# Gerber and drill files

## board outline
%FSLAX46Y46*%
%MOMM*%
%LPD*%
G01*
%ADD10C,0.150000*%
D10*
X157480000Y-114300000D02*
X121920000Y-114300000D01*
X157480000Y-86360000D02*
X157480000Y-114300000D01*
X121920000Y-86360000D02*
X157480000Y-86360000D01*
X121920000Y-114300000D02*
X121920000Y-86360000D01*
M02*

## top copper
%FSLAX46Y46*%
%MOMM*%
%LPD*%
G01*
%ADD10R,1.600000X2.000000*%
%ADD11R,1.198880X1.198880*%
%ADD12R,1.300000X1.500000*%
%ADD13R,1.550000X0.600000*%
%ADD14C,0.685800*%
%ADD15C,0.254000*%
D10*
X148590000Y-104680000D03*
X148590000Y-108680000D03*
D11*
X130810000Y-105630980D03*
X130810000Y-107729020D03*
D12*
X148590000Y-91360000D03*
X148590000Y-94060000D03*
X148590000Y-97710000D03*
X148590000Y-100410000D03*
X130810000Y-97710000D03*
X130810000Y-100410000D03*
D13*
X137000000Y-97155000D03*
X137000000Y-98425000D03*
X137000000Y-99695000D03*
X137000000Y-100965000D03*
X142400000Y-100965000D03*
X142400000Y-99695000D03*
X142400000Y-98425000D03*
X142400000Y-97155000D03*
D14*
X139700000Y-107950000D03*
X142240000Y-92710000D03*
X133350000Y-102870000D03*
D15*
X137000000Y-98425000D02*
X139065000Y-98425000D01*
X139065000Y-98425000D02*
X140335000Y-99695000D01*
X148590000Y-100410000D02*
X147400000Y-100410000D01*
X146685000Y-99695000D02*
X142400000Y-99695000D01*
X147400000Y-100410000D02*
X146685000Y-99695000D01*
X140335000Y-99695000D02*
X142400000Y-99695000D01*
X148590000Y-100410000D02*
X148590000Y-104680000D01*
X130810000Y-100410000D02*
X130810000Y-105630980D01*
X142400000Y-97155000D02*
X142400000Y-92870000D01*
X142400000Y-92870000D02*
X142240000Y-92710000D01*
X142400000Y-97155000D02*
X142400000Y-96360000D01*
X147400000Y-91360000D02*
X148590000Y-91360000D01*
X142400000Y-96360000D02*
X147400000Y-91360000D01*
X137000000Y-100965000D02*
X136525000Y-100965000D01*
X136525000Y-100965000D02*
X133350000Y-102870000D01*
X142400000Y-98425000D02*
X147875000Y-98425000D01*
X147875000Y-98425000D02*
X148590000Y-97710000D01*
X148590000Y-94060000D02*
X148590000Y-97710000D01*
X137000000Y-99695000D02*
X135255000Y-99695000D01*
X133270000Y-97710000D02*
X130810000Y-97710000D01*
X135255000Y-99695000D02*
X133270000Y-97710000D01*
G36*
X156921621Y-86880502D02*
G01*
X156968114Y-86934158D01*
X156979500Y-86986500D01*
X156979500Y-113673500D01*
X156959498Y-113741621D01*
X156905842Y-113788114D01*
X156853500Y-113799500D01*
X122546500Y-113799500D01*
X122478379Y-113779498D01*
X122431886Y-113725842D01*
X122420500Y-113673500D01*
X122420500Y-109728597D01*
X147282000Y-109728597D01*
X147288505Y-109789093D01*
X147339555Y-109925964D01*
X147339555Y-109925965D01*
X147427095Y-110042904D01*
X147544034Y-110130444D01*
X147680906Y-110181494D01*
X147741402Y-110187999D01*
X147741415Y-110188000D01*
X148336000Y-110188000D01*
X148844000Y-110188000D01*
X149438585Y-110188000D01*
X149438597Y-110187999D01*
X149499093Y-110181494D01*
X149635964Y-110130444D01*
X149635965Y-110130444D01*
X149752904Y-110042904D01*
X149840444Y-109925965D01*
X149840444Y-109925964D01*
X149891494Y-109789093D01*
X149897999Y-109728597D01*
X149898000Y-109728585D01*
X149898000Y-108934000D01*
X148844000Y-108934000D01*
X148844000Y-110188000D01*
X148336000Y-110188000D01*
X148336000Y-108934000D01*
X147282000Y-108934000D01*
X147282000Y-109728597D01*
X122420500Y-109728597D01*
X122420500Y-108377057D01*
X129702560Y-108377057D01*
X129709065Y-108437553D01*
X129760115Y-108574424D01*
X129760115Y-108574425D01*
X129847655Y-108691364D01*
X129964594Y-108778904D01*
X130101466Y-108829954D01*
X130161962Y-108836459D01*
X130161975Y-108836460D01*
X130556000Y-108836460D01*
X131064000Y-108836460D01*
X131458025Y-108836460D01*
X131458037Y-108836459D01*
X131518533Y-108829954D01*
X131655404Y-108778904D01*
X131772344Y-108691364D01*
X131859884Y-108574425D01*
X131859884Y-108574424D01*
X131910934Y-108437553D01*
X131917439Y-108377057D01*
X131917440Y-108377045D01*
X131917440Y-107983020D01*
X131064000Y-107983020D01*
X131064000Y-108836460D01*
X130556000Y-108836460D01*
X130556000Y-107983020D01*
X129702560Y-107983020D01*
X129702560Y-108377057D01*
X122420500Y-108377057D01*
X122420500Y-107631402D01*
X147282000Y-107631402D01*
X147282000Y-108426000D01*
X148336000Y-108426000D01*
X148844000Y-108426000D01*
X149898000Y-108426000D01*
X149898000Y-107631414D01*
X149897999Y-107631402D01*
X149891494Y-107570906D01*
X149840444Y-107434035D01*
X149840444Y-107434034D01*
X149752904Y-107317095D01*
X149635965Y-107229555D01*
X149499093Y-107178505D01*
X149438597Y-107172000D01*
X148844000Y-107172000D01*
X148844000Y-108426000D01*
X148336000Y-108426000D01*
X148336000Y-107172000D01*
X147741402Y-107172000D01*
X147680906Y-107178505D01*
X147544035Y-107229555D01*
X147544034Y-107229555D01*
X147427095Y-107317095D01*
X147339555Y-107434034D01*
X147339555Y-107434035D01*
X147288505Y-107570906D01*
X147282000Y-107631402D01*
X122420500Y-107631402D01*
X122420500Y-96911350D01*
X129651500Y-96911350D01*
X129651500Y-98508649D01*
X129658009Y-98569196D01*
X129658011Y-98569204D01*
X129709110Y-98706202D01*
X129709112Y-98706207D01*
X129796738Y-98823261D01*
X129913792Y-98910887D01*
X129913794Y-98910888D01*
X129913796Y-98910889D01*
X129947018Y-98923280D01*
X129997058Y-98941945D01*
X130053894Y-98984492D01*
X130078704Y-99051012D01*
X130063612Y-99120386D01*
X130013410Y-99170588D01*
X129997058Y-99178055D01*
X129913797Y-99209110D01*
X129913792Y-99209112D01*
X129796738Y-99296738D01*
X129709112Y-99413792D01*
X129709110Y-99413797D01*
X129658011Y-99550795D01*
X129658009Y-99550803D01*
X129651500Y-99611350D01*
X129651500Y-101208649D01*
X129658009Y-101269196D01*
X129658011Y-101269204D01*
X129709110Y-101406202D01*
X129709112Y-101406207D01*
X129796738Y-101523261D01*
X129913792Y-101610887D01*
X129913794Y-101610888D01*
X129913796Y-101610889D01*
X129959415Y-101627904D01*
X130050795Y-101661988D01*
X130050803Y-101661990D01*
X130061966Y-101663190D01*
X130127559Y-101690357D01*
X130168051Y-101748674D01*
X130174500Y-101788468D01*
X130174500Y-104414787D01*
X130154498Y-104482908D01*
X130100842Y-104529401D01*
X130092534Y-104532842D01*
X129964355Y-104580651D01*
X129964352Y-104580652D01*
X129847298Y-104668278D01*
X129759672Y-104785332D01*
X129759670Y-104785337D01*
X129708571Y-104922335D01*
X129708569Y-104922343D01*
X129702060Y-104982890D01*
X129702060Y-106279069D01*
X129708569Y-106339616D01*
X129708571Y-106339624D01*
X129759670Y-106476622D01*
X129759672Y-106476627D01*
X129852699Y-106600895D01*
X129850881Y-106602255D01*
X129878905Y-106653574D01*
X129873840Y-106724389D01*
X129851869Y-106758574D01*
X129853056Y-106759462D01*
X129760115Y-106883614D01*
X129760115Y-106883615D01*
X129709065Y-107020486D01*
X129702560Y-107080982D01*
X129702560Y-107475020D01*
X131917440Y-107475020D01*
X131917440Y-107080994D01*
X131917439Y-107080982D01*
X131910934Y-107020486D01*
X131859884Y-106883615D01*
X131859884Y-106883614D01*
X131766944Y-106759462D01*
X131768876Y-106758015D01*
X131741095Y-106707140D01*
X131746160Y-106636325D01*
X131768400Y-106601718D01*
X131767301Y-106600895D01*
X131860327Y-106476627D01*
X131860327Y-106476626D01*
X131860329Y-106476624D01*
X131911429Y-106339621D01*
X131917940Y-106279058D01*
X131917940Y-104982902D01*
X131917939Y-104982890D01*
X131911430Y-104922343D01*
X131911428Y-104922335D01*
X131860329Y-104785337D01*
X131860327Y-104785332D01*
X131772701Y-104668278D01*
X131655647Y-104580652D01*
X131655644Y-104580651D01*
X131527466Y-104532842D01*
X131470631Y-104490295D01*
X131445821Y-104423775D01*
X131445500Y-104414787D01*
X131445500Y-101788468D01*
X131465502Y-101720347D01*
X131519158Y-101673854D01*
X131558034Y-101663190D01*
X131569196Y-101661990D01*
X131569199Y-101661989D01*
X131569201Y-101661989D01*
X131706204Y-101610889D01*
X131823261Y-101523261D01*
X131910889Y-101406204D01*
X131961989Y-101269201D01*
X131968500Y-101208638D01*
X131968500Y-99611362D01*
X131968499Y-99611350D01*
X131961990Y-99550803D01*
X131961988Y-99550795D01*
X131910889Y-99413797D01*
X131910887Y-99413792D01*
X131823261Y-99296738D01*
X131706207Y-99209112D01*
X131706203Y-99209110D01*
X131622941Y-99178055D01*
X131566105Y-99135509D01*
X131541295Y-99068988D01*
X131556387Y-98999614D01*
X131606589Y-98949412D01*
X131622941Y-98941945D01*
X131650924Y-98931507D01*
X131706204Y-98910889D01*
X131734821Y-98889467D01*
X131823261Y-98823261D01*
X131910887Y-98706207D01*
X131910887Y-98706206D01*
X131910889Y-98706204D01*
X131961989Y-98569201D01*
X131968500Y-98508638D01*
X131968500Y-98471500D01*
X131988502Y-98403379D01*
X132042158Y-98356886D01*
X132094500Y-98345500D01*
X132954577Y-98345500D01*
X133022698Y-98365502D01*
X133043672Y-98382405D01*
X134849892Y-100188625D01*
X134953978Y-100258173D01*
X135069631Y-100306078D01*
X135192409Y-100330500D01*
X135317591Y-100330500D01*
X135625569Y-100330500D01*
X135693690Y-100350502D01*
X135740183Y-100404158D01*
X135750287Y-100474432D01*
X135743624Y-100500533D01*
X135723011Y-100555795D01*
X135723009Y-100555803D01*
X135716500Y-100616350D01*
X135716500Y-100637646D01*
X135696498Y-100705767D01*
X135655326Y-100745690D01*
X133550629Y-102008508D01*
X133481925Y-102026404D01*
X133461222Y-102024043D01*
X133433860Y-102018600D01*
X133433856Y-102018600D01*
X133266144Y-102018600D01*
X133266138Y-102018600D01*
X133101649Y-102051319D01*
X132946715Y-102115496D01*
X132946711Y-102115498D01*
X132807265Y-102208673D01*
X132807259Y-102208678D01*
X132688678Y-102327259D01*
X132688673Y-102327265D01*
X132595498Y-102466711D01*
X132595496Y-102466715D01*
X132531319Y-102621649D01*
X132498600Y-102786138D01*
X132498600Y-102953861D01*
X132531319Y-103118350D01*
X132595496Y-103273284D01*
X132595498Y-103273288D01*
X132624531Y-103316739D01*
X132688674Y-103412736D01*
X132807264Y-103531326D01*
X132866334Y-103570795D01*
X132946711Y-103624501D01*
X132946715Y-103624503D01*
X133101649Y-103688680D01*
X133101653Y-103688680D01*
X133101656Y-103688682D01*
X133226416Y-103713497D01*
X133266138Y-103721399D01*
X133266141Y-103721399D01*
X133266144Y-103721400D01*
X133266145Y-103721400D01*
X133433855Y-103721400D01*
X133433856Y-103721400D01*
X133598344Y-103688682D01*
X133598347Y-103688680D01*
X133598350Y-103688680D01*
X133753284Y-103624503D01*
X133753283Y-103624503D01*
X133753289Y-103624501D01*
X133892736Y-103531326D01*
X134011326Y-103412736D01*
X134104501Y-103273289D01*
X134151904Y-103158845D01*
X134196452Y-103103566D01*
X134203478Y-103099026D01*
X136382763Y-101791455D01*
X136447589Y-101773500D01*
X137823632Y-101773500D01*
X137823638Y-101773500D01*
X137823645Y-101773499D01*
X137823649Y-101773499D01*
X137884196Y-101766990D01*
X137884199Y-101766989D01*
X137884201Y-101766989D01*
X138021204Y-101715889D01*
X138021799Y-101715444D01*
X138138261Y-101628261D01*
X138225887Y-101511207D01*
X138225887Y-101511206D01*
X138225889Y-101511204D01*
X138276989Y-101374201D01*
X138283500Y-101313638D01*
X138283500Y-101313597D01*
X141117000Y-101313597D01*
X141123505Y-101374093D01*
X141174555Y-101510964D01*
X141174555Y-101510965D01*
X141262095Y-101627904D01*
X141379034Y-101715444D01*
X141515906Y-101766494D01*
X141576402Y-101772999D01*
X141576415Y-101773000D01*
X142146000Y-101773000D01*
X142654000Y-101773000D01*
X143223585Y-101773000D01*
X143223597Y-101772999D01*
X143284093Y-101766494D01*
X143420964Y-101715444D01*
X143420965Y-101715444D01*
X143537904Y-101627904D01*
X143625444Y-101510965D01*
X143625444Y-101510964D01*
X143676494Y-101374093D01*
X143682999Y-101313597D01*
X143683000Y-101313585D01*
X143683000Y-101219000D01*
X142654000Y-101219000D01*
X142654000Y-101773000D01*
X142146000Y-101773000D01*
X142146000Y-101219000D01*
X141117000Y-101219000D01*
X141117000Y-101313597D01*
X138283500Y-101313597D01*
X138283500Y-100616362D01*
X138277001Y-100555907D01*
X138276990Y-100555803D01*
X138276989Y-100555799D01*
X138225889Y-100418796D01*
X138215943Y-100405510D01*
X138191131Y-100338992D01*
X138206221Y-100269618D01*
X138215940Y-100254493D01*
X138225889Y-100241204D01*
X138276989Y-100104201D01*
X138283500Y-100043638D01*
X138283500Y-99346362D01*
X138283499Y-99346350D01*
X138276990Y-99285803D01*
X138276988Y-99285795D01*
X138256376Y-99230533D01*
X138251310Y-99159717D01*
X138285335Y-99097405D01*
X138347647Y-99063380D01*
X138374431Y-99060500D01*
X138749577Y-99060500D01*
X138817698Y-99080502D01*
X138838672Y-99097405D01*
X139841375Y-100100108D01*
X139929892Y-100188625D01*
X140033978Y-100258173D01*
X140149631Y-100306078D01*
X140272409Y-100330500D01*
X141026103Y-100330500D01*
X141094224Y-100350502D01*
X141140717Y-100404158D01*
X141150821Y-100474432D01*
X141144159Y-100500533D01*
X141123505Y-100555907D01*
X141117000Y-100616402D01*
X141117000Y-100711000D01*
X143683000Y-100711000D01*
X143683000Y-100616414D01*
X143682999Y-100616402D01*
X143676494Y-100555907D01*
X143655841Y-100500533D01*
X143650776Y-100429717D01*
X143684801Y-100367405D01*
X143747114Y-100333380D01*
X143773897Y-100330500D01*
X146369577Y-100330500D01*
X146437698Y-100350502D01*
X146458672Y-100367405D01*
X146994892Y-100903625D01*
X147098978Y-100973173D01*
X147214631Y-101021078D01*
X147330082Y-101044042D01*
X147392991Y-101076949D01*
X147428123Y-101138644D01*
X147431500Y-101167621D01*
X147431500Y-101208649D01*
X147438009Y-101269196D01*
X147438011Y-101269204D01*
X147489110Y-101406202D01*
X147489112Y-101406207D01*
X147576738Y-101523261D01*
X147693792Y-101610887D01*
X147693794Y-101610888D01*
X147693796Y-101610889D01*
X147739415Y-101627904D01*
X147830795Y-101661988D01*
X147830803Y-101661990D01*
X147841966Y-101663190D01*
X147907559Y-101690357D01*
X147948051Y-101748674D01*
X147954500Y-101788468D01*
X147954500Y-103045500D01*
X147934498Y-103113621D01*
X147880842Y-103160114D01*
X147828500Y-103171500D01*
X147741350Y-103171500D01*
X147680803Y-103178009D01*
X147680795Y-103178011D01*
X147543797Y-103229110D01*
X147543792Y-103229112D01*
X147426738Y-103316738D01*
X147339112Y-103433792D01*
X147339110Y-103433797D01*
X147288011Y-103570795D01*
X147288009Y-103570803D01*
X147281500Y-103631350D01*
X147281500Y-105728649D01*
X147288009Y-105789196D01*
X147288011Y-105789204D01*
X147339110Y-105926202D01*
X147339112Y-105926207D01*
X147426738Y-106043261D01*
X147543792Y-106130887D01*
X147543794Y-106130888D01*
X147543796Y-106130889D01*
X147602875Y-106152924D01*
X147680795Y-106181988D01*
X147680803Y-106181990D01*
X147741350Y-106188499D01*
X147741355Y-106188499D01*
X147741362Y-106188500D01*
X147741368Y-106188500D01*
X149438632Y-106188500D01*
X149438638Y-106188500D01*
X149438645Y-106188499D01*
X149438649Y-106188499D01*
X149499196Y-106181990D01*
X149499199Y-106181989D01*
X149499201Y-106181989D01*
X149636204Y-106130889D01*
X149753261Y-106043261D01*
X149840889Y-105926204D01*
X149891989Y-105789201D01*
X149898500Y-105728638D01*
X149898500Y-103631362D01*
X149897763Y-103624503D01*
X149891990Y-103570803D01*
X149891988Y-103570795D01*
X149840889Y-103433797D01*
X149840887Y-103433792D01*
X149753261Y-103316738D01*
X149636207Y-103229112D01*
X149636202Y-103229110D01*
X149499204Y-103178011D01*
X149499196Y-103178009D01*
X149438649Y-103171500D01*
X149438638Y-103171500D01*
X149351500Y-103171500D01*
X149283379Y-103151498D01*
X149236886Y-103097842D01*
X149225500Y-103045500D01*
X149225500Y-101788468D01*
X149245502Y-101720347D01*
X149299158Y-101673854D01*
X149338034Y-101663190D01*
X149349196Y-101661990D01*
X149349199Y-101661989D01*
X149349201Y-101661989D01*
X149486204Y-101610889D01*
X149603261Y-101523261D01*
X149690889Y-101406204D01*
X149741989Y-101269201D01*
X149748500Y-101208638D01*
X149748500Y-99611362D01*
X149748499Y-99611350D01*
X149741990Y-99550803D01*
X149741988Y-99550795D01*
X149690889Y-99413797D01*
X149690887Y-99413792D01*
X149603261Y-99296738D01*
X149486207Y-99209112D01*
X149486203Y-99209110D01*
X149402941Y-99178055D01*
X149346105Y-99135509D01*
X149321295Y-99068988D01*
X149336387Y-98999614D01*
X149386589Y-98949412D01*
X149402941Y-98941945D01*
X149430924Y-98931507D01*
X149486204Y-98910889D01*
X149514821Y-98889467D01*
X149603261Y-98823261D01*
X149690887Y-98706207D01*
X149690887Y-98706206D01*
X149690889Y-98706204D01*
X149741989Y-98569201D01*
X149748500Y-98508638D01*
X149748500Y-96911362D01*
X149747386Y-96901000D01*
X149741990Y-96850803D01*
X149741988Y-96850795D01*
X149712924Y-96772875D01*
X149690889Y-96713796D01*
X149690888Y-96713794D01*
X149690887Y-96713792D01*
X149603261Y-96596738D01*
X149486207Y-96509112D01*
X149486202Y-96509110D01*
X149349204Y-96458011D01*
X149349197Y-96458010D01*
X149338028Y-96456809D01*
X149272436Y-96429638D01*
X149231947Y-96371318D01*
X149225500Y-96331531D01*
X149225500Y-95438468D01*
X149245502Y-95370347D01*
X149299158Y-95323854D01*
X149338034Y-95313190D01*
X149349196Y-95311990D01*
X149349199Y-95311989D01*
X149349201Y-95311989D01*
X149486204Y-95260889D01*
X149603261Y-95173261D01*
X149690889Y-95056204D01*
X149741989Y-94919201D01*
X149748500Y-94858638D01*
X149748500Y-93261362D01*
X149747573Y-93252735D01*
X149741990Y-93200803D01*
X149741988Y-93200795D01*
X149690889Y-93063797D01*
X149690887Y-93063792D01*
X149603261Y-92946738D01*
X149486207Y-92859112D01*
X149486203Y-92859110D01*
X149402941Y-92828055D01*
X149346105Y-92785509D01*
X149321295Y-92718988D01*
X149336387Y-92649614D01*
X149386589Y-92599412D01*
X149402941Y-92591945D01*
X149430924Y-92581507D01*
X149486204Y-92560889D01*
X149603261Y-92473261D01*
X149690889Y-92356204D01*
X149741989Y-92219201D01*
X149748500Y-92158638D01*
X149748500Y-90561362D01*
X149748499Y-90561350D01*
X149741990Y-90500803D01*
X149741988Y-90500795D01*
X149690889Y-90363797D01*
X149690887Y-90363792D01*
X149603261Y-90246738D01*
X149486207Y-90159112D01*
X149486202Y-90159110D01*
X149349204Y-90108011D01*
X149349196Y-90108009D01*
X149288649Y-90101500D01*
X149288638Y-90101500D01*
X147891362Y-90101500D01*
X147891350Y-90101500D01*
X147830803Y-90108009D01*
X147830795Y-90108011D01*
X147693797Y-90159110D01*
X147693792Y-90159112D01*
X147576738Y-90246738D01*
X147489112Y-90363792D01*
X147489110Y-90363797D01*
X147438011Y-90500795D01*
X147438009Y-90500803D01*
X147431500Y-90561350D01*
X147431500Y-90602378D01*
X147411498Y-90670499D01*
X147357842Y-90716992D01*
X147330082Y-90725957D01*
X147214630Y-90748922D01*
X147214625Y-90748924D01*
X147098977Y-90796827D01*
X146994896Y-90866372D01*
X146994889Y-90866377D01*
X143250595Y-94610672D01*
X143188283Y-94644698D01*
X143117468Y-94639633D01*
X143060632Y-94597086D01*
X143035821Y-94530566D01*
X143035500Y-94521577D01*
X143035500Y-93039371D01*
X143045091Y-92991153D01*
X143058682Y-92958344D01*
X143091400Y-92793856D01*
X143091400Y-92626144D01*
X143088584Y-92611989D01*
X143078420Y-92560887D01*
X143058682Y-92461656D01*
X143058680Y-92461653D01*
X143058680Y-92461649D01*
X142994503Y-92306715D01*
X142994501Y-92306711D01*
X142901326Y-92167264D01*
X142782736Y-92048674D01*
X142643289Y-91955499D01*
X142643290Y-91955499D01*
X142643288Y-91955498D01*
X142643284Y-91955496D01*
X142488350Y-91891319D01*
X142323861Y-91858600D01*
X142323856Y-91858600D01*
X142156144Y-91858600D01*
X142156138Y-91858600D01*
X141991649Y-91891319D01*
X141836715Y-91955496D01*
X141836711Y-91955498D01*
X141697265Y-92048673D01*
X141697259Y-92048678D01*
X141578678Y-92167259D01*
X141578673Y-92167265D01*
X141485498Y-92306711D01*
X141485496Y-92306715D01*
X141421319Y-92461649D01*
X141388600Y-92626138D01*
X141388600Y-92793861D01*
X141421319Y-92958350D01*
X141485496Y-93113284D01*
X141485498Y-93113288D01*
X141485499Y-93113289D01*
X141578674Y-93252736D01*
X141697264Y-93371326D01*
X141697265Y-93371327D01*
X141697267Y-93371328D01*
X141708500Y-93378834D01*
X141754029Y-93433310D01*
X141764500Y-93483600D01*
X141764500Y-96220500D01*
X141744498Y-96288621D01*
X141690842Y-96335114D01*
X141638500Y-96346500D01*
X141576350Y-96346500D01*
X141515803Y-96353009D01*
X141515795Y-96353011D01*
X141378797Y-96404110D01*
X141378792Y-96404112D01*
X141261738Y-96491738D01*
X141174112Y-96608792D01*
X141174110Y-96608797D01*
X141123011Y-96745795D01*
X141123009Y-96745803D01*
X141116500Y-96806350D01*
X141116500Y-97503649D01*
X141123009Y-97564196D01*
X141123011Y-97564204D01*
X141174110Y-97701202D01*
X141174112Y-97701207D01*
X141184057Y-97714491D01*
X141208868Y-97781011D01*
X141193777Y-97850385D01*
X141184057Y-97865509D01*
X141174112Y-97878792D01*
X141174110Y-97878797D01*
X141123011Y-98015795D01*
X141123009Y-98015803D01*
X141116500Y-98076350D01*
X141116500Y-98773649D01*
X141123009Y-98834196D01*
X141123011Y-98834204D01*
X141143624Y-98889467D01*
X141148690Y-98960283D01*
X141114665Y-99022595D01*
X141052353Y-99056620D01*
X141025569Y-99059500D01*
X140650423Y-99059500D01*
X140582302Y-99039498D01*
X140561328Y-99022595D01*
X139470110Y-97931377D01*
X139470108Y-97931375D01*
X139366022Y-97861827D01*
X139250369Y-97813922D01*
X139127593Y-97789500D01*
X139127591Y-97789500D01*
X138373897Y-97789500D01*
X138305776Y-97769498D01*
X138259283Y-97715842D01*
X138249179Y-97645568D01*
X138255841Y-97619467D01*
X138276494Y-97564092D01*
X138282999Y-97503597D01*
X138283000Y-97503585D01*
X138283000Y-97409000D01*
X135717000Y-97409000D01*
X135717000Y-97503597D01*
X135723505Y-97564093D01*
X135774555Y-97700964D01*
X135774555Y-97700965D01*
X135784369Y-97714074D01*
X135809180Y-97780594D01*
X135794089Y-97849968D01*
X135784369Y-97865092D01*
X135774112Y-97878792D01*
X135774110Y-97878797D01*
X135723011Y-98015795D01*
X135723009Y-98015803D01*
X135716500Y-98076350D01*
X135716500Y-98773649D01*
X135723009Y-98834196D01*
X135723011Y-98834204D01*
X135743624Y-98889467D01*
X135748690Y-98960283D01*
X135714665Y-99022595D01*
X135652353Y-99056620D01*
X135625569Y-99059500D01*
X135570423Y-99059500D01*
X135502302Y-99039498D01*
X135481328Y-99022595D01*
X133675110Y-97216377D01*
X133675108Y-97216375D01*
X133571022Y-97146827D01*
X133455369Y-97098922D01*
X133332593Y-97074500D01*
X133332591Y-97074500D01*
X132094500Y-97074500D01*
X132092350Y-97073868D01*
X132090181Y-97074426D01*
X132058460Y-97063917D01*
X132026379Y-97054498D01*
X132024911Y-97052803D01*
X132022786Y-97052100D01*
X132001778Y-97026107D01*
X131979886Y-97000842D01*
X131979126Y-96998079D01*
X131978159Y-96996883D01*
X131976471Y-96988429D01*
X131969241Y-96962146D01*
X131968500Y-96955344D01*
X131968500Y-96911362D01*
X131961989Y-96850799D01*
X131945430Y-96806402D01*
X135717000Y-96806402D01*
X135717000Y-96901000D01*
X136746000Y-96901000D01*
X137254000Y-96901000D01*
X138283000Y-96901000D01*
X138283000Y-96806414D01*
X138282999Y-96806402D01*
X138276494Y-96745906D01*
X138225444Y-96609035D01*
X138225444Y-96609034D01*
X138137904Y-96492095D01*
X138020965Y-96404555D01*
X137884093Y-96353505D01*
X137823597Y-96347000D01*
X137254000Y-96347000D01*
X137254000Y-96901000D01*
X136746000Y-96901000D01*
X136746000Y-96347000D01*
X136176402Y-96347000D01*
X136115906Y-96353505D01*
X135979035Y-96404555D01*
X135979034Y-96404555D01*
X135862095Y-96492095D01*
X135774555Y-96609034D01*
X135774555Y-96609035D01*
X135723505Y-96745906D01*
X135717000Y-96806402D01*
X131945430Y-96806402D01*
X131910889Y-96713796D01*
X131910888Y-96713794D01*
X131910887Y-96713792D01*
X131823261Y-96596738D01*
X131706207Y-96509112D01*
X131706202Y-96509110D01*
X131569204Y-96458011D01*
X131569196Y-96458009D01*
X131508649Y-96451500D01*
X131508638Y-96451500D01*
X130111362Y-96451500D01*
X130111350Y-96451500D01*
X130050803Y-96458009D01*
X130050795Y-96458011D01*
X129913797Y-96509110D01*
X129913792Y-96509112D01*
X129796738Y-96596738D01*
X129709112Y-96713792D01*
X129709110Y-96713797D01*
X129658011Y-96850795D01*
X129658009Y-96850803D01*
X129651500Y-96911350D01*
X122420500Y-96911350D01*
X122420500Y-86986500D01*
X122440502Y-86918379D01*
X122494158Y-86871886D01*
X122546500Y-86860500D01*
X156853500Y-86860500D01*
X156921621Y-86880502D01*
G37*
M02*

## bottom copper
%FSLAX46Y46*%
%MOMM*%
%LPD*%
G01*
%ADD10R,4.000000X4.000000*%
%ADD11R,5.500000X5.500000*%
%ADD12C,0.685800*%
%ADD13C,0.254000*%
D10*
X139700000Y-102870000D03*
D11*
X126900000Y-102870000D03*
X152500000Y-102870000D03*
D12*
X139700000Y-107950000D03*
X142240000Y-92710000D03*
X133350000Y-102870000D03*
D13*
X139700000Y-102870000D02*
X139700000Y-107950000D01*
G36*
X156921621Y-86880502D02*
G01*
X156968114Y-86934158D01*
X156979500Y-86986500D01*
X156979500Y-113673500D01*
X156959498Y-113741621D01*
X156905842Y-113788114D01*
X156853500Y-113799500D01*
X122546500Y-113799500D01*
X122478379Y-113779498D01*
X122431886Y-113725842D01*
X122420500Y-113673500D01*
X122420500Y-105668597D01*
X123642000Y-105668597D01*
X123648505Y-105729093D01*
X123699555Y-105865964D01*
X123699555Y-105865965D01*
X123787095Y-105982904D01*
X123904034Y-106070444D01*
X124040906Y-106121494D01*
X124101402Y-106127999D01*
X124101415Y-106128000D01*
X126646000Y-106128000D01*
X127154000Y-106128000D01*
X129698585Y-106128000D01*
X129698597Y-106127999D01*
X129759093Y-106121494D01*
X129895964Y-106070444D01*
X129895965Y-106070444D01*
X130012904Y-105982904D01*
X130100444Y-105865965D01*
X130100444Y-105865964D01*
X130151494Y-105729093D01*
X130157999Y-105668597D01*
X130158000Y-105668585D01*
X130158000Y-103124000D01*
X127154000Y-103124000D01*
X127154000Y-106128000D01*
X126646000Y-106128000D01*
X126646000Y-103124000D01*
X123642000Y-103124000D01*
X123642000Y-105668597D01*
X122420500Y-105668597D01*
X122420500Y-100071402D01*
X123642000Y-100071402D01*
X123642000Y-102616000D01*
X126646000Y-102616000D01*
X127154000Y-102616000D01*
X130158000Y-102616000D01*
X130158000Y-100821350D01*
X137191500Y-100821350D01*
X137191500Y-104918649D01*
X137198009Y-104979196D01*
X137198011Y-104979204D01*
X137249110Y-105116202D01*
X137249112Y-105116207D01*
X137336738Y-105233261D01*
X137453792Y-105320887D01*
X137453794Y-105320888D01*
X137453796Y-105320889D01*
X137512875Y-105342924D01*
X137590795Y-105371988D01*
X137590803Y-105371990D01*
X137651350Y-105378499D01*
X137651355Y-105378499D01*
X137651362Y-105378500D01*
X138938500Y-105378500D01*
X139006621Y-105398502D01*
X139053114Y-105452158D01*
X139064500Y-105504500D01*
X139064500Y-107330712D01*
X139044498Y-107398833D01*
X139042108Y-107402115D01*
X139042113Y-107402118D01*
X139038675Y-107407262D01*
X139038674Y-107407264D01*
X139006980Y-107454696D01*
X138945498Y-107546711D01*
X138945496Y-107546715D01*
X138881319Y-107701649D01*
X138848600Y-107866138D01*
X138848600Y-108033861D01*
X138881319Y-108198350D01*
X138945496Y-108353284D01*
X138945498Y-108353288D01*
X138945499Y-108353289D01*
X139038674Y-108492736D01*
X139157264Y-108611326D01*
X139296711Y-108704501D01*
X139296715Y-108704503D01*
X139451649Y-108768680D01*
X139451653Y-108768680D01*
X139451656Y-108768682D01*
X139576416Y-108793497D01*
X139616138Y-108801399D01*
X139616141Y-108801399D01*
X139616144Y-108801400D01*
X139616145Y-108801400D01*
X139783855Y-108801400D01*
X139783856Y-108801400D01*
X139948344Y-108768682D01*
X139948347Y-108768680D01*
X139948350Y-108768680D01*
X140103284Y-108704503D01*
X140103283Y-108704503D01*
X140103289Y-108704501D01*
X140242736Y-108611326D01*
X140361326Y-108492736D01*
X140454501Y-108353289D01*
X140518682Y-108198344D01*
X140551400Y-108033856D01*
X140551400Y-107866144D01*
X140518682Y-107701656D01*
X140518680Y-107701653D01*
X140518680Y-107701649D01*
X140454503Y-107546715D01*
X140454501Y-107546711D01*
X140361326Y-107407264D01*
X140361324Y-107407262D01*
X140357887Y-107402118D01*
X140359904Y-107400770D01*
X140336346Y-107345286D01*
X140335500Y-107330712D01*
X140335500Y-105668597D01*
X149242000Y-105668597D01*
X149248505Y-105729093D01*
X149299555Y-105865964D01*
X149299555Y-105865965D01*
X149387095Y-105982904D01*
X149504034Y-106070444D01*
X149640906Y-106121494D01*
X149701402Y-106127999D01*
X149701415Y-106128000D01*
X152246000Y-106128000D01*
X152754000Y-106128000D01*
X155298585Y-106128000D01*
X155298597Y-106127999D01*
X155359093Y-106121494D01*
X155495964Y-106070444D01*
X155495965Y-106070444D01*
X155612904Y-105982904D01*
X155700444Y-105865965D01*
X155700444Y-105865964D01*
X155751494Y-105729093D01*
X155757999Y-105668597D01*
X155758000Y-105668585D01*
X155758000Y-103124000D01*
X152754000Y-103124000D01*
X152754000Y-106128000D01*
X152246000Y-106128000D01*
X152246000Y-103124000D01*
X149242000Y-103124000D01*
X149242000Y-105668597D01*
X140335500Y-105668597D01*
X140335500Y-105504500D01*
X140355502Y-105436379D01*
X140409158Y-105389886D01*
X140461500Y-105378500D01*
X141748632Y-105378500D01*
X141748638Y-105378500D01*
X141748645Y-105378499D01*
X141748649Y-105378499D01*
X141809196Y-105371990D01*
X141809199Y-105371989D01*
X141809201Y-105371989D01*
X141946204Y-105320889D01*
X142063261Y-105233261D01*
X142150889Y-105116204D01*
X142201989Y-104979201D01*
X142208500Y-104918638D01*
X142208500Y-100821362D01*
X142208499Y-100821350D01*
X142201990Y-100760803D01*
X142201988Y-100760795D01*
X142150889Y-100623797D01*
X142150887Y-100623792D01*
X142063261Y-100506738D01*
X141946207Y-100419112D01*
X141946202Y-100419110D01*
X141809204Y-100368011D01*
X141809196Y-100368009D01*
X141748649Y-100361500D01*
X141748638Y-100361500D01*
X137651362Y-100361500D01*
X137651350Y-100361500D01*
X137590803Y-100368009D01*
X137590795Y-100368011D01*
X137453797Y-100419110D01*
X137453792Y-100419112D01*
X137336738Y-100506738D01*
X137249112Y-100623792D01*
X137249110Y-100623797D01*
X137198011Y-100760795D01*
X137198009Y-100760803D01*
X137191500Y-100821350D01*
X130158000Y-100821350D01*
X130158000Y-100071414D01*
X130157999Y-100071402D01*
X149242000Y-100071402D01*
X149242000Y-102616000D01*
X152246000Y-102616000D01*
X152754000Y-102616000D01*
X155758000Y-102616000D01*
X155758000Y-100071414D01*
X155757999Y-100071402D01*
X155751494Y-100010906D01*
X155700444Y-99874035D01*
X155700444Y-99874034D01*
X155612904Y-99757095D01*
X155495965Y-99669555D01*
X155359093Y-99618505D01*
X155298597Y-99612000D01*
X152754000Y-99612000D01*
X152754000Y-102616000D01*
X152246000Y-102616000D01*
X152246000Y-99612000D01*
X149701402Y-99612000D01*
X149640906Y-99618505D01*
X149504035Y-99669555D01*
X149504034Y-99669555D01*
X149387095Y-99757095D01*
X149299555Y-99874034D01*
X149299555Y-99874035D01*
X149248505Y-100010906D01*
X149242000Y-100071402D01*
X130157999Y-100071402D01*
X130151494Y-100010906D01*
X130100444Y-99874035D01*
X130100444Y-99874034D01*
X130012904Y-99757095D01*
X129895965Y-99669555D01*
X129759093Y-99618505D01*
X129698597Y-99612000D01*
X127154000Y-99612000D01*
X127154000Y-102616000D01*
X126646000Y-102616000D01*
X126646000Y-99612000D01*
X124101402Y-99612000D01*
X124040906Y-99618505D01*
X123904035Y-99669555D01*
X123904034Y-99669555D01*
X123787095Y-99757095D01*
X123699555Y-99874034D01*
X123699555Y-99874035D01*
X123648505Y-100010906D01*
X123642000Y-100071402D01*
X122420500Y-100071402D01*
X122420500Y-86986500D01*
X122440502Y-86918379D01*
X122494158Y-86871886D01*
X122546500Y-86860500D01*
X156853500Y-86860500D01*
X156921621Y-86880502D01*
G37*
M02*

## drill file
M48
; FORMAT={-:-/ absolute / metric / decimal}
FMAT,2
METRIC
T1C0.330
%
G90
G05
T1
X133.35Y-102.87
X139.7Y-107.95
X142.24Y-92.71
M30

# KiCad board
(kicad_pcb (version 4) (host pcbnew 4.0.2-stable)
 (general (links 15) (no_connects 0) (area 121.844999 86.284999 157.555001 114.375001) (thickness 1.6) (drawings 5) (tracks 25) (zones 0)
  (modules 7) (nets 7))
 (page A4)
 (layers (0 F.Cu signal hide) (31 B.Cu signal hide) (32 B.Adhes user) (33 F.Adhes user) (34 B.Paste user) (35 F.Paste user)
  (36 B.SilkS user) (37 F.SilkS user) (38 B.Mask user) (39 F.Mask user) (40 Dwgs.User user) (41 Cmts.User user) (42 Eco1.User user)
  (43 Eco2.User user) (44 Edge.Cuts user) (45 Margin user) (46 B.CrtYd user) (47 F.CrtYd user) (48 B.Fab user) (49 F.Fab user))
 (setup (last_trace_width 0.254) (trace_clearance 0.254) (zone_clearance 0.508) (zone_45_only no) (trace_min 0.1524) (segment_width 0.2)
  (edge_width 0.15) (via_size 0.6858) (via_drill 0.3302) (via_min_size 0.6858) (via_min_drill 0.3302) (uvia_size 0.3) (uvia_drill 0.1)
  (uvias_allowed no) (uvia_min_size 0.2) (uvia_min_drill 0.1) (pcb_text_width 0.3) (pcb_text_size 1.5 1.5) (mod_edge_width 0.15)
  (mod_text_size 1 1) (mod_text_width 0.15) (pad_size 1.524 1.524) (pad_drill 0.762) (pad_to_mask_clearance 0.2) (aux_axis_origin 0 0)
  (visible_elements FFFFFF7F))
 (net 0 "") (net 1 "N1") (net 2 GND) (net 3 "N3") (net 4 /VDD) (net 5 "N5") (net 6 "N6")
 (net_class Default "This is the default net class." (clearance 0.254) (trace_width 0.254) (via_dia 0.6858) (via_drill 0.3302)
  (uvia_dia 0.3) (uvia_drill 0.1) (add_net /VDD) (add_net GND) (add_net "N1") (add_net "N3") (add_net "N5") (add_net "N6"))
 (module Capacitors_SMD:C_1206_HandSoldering (layer F.Cu) (at 148.59 106.68 270)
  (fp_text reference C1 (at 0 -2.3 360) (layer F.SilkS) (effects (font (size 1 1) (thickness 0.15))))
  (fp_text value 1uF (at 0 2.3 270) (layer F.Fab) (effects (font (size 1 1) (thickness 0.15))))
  (pad 1 smd rect (at -2 0 270) (size 2 1.6) (layers F.Cu F.Paste F.Mask) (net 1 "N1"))
  (pad 2 smd rect (at 2 0 270) (size 2 1.6) (layers F.Cu F.Paste F.Mask) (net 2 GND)))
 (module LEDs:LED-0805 (layer F.Cu) (at 130.81 106.68 90)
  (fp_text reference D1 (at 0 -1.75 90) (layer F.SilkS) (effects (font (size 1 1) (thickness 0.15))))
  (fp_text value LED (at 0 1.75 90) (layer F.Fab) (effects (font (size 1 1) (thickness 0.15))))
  (pad 2 smd rect (at 1.04902 0 270) (size 1.19888 1.19888) (layers F.Cu F.Paste F.Mask) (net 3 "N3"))
  (pad 1 smd rect (at -1.04902 0 270) (size 1.19888 1.19888) (layers F.Cu F.Paste F.Mask) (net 2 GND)))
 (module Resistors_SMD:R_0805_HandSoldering (layer F.Cu) (at 148.59 92.71 270)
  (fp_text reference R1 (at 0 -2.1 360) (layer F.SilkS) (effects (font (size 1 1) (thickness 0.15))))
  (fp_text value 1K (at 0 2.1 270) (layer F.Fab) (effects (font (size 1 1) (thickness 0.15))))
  (pad 1 smd rect (at -1.35 0 270) (size 1.5 1.3) (layers F.Cu F.Paste F.Mask) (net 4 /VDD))
  (pad 2 smd rect (at 1.35 0 270) (size 1.5 1.3) (layers F.Cu F.Paste F.Mask) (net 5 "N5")))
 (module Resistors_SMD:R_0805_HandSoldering (layer F.Cu) (at 148.59 99.06 270)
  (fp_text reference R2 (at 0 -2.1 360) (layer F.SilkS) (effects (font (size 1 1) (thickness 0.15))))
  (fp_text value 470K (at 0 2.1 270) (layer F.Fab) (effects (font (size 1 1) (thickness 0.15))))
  (pad 1 smd rect (at -1.35 0 270) (size 1.5 1.3) (layers F.Cu F.Paste F.Mask) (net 5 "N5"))
  (pad 2 smd rect (at 1.35 0 270) (size 1.5 1.3) (layers F.Cu F.Paste F.Mask) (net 1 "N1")))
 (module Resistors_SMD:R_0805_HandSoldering (layer F.Cu) (at 130.81 99.06 270)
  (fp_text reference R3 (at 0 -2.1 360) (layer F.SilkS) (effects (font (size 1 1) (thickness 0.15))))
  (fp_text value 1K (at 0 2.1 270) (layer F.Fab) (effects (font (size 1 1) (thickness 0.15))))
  (pad 1 smd rect (at -1.35 0 270) (size 1.5 1.3) (layers F.Cu F.Paste F.Mask) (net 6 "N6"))
  (pad 2 smd rect (at 1.35 0 270) (size 1.5 1.3) (layers F.Cu F.Paste F.Mask) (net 3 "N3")))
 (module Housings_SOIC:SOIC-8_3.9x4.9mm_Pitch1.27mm (layer F.Cu) (at 139.7 99.06)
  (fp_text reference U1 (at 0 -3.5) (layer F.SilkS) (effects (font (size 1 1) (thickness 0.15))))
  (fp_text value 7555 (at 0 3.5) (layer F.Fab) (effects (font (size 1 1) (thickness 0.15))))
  (pad 1 smd rect (at -2.7 -1.905) (size 1.55 0.6) (layers F.Cu F.Paste F.Mask) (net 2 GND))
  (pad 2 smd rect (at -2.7 -0.635) (size 1.55 0.6) (layers F.Cu F.Paste F.Mask) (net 1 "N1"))
  (pad 3 smd rect (at -2.7 0.635) (size 1.55 0.6) (layers F.Cu F.Paste F.Mask) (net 6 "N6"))
  (pad 4 smd rect (at -2.7 1.905) (size 1.55 0.6) (layers F.Cu F.Paste F.Mask) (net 4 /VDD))
  (pad 5 smd rect (at 2.7 1.905) (size 1.55 0.6) (layers F.Cu F.Paste F.Mask) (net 2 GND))
  (pad 6 smd rect (at 2.7 0.635) (size 1.55 0.6) (layers F.Cu F.Paste F.Mask) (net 1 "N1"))
  (pad 7 smd rect (at 2.7 -0.635) (size 1.55 0.6) (layers F.Cu F.Paste F.Mask) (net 5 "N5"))
  (pad 8 smd rect (at 2.7 -1.905) (size 1.55 0.6) (layers F.Cu F.Paste F.Mask) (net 4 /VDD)))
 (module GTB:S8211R (layer B.Cu) (at 139.7 102.87)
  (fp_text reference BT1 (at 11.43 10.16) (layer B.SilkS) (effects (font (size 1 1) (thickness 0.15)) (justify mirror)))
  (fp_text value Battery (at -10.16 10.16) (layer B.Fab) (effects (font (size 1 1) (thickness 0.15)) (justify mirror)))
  (pad 2 smd rect (at 0 0) (size 4 4) (layers B.Cu B.Paste B.Mask) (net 2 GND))
  (pad 1 smd rect (at -12.8 0) (size 5.5 5.5) (layers B.Cu B.Paste B.Mask) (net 4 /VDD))
  (pad 1 smd rect (at 12.8 0) (size 5.5 5.5) (layers B.Cu B.Paste B.Mask) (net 4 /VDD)))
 (gr_line (start 157.48 114.3) (end 121.92 114.3) (angle 90) (layer Edge.Cuts) (width 0.15))
 (gr_line (start 157.48 86.36) (end 157.48 114.3) (angle 90) (layer Edge.Cuts) (width 0.15))
 (gr_line (start 121.92 86.36) (end 157.48 86.36) (angle 90) (layer Edge.Cuts) (width 0.15))
 (gr_line (start 121.92 114.3) (end 121.92 86.36) (angle 90) (layer Edge.Cuts) (width 0.15))
 (segment (start 137 98.425) (end 139.065 98.425) (width 0.254) (layer F.Cu) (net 1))
 (segment (start 139.065 98.425) (end 140.335 99.695) (width 0.254) (layer F.Cu) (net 1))
 (segment (start 148.59 100.41) (end 147.4 100.41) (width 0.254) (layer F.Cu) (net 1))
 (segment (start 146.685 99.695) (end 142.4 99.695) (width 0.254) (layer F.Cu) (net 1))
 (segment (start 147.4 100.41) (end 146.685 99.695) (width 0.254) (layer F.Cu) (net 1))
 (segment (start 140.335 99.695) (end 142.4 99.695) (width 0.254) (layer F.Cu) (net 1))
 (segment (start 148.59 100.41) (end 148.59 104.68) (width 0.254) (layer F.Cu) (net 1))
 (segment (start 139.7 102.87) (end 139.7 107.95) (width 0.254) (layer B.Cu) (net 2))
 (via (at 139.7 107.95) (size 0.6858) (drill 0.3302) (layers F.Cu B.Cu) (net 2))
 (segment (start 130.81 100.41) (end 130.81 105.63098) (width 0.254) (layer F.Cu) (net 3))
 (segment (start 142.4 97.155) (end 142.4 92.87) (width 0.254) (layer F.Cu) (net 4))
 (via (at 142.24 92.71) (size 0.6858) (drill 0.3302) (layers F.Cu B.Cu) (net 4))
 (segment (start 142.4 92.87) (end 142.24 92.71) (width 0.254) (layer F.Cu) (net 4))
 (segment (start 142.4 97.155) (end 142.4 96.36) (width 0.254) (layer F.Cu) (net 4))
 (segment (start 147.4 91.36) (end 148.59 91.36) (width 0.254) (layer F.Cu) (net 4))
 (segment (start 142.4 96.36) (end 147.4 91.36) (width 0.254) (layer F.Cu) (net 4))
 (segment (start 137 100.965) (end 136.525 100.965) (width 0.254) (layer F.Cu) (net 4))
 (segment (start 136.525 100.965) (end 133.35 102.87) (width 0.254) (layer F.Cu) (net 4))
 (via (at 133.35 102.87) (size 0.6858) (drill 0.3302) (layers F.Cu B.Cu) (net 4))
 (segment (start 142.4 98.425) (end 147.875 98.425) (width 0.254) (layer F.Cu) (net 5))
 (segment (start 147.875 98.425) (end 148.59 97.71) (width 0.254) (layer F.Cu) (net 5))
 (segment (start 148.59 94.06) (end 148.59 97.71) (width 0.254) (layer F.Cu) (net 5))
 (segment (start 137 99.695) (end 135.255 99.695) (width 0.254) (layer F.Cu) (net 6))
 (segment (start 133.27 97.71) (end 130.81 97.71) (width 0.254) (layer F.Cu) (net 6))
 (segment (start 135.255 99.695) (end 133.27 97.71) (width 0.254) (layer F.Cu) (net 6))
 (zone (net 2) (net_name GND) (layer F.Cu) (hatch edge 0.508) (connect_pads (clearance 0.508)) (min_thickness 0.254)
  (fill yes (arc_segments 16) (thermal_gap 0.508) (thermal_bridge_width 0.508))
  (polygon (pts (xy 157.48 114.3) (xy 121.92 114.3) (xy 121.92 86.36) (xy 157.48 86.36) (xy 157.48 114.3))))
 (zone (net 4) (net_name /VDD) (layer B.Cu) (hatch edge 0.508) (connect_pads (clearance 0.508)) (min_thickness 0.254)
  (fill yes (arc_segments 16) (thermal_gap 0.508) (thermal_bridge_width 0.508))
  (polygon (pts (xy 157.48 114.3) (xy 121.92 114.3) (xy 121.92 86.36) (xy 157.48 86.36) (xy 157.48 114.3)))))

